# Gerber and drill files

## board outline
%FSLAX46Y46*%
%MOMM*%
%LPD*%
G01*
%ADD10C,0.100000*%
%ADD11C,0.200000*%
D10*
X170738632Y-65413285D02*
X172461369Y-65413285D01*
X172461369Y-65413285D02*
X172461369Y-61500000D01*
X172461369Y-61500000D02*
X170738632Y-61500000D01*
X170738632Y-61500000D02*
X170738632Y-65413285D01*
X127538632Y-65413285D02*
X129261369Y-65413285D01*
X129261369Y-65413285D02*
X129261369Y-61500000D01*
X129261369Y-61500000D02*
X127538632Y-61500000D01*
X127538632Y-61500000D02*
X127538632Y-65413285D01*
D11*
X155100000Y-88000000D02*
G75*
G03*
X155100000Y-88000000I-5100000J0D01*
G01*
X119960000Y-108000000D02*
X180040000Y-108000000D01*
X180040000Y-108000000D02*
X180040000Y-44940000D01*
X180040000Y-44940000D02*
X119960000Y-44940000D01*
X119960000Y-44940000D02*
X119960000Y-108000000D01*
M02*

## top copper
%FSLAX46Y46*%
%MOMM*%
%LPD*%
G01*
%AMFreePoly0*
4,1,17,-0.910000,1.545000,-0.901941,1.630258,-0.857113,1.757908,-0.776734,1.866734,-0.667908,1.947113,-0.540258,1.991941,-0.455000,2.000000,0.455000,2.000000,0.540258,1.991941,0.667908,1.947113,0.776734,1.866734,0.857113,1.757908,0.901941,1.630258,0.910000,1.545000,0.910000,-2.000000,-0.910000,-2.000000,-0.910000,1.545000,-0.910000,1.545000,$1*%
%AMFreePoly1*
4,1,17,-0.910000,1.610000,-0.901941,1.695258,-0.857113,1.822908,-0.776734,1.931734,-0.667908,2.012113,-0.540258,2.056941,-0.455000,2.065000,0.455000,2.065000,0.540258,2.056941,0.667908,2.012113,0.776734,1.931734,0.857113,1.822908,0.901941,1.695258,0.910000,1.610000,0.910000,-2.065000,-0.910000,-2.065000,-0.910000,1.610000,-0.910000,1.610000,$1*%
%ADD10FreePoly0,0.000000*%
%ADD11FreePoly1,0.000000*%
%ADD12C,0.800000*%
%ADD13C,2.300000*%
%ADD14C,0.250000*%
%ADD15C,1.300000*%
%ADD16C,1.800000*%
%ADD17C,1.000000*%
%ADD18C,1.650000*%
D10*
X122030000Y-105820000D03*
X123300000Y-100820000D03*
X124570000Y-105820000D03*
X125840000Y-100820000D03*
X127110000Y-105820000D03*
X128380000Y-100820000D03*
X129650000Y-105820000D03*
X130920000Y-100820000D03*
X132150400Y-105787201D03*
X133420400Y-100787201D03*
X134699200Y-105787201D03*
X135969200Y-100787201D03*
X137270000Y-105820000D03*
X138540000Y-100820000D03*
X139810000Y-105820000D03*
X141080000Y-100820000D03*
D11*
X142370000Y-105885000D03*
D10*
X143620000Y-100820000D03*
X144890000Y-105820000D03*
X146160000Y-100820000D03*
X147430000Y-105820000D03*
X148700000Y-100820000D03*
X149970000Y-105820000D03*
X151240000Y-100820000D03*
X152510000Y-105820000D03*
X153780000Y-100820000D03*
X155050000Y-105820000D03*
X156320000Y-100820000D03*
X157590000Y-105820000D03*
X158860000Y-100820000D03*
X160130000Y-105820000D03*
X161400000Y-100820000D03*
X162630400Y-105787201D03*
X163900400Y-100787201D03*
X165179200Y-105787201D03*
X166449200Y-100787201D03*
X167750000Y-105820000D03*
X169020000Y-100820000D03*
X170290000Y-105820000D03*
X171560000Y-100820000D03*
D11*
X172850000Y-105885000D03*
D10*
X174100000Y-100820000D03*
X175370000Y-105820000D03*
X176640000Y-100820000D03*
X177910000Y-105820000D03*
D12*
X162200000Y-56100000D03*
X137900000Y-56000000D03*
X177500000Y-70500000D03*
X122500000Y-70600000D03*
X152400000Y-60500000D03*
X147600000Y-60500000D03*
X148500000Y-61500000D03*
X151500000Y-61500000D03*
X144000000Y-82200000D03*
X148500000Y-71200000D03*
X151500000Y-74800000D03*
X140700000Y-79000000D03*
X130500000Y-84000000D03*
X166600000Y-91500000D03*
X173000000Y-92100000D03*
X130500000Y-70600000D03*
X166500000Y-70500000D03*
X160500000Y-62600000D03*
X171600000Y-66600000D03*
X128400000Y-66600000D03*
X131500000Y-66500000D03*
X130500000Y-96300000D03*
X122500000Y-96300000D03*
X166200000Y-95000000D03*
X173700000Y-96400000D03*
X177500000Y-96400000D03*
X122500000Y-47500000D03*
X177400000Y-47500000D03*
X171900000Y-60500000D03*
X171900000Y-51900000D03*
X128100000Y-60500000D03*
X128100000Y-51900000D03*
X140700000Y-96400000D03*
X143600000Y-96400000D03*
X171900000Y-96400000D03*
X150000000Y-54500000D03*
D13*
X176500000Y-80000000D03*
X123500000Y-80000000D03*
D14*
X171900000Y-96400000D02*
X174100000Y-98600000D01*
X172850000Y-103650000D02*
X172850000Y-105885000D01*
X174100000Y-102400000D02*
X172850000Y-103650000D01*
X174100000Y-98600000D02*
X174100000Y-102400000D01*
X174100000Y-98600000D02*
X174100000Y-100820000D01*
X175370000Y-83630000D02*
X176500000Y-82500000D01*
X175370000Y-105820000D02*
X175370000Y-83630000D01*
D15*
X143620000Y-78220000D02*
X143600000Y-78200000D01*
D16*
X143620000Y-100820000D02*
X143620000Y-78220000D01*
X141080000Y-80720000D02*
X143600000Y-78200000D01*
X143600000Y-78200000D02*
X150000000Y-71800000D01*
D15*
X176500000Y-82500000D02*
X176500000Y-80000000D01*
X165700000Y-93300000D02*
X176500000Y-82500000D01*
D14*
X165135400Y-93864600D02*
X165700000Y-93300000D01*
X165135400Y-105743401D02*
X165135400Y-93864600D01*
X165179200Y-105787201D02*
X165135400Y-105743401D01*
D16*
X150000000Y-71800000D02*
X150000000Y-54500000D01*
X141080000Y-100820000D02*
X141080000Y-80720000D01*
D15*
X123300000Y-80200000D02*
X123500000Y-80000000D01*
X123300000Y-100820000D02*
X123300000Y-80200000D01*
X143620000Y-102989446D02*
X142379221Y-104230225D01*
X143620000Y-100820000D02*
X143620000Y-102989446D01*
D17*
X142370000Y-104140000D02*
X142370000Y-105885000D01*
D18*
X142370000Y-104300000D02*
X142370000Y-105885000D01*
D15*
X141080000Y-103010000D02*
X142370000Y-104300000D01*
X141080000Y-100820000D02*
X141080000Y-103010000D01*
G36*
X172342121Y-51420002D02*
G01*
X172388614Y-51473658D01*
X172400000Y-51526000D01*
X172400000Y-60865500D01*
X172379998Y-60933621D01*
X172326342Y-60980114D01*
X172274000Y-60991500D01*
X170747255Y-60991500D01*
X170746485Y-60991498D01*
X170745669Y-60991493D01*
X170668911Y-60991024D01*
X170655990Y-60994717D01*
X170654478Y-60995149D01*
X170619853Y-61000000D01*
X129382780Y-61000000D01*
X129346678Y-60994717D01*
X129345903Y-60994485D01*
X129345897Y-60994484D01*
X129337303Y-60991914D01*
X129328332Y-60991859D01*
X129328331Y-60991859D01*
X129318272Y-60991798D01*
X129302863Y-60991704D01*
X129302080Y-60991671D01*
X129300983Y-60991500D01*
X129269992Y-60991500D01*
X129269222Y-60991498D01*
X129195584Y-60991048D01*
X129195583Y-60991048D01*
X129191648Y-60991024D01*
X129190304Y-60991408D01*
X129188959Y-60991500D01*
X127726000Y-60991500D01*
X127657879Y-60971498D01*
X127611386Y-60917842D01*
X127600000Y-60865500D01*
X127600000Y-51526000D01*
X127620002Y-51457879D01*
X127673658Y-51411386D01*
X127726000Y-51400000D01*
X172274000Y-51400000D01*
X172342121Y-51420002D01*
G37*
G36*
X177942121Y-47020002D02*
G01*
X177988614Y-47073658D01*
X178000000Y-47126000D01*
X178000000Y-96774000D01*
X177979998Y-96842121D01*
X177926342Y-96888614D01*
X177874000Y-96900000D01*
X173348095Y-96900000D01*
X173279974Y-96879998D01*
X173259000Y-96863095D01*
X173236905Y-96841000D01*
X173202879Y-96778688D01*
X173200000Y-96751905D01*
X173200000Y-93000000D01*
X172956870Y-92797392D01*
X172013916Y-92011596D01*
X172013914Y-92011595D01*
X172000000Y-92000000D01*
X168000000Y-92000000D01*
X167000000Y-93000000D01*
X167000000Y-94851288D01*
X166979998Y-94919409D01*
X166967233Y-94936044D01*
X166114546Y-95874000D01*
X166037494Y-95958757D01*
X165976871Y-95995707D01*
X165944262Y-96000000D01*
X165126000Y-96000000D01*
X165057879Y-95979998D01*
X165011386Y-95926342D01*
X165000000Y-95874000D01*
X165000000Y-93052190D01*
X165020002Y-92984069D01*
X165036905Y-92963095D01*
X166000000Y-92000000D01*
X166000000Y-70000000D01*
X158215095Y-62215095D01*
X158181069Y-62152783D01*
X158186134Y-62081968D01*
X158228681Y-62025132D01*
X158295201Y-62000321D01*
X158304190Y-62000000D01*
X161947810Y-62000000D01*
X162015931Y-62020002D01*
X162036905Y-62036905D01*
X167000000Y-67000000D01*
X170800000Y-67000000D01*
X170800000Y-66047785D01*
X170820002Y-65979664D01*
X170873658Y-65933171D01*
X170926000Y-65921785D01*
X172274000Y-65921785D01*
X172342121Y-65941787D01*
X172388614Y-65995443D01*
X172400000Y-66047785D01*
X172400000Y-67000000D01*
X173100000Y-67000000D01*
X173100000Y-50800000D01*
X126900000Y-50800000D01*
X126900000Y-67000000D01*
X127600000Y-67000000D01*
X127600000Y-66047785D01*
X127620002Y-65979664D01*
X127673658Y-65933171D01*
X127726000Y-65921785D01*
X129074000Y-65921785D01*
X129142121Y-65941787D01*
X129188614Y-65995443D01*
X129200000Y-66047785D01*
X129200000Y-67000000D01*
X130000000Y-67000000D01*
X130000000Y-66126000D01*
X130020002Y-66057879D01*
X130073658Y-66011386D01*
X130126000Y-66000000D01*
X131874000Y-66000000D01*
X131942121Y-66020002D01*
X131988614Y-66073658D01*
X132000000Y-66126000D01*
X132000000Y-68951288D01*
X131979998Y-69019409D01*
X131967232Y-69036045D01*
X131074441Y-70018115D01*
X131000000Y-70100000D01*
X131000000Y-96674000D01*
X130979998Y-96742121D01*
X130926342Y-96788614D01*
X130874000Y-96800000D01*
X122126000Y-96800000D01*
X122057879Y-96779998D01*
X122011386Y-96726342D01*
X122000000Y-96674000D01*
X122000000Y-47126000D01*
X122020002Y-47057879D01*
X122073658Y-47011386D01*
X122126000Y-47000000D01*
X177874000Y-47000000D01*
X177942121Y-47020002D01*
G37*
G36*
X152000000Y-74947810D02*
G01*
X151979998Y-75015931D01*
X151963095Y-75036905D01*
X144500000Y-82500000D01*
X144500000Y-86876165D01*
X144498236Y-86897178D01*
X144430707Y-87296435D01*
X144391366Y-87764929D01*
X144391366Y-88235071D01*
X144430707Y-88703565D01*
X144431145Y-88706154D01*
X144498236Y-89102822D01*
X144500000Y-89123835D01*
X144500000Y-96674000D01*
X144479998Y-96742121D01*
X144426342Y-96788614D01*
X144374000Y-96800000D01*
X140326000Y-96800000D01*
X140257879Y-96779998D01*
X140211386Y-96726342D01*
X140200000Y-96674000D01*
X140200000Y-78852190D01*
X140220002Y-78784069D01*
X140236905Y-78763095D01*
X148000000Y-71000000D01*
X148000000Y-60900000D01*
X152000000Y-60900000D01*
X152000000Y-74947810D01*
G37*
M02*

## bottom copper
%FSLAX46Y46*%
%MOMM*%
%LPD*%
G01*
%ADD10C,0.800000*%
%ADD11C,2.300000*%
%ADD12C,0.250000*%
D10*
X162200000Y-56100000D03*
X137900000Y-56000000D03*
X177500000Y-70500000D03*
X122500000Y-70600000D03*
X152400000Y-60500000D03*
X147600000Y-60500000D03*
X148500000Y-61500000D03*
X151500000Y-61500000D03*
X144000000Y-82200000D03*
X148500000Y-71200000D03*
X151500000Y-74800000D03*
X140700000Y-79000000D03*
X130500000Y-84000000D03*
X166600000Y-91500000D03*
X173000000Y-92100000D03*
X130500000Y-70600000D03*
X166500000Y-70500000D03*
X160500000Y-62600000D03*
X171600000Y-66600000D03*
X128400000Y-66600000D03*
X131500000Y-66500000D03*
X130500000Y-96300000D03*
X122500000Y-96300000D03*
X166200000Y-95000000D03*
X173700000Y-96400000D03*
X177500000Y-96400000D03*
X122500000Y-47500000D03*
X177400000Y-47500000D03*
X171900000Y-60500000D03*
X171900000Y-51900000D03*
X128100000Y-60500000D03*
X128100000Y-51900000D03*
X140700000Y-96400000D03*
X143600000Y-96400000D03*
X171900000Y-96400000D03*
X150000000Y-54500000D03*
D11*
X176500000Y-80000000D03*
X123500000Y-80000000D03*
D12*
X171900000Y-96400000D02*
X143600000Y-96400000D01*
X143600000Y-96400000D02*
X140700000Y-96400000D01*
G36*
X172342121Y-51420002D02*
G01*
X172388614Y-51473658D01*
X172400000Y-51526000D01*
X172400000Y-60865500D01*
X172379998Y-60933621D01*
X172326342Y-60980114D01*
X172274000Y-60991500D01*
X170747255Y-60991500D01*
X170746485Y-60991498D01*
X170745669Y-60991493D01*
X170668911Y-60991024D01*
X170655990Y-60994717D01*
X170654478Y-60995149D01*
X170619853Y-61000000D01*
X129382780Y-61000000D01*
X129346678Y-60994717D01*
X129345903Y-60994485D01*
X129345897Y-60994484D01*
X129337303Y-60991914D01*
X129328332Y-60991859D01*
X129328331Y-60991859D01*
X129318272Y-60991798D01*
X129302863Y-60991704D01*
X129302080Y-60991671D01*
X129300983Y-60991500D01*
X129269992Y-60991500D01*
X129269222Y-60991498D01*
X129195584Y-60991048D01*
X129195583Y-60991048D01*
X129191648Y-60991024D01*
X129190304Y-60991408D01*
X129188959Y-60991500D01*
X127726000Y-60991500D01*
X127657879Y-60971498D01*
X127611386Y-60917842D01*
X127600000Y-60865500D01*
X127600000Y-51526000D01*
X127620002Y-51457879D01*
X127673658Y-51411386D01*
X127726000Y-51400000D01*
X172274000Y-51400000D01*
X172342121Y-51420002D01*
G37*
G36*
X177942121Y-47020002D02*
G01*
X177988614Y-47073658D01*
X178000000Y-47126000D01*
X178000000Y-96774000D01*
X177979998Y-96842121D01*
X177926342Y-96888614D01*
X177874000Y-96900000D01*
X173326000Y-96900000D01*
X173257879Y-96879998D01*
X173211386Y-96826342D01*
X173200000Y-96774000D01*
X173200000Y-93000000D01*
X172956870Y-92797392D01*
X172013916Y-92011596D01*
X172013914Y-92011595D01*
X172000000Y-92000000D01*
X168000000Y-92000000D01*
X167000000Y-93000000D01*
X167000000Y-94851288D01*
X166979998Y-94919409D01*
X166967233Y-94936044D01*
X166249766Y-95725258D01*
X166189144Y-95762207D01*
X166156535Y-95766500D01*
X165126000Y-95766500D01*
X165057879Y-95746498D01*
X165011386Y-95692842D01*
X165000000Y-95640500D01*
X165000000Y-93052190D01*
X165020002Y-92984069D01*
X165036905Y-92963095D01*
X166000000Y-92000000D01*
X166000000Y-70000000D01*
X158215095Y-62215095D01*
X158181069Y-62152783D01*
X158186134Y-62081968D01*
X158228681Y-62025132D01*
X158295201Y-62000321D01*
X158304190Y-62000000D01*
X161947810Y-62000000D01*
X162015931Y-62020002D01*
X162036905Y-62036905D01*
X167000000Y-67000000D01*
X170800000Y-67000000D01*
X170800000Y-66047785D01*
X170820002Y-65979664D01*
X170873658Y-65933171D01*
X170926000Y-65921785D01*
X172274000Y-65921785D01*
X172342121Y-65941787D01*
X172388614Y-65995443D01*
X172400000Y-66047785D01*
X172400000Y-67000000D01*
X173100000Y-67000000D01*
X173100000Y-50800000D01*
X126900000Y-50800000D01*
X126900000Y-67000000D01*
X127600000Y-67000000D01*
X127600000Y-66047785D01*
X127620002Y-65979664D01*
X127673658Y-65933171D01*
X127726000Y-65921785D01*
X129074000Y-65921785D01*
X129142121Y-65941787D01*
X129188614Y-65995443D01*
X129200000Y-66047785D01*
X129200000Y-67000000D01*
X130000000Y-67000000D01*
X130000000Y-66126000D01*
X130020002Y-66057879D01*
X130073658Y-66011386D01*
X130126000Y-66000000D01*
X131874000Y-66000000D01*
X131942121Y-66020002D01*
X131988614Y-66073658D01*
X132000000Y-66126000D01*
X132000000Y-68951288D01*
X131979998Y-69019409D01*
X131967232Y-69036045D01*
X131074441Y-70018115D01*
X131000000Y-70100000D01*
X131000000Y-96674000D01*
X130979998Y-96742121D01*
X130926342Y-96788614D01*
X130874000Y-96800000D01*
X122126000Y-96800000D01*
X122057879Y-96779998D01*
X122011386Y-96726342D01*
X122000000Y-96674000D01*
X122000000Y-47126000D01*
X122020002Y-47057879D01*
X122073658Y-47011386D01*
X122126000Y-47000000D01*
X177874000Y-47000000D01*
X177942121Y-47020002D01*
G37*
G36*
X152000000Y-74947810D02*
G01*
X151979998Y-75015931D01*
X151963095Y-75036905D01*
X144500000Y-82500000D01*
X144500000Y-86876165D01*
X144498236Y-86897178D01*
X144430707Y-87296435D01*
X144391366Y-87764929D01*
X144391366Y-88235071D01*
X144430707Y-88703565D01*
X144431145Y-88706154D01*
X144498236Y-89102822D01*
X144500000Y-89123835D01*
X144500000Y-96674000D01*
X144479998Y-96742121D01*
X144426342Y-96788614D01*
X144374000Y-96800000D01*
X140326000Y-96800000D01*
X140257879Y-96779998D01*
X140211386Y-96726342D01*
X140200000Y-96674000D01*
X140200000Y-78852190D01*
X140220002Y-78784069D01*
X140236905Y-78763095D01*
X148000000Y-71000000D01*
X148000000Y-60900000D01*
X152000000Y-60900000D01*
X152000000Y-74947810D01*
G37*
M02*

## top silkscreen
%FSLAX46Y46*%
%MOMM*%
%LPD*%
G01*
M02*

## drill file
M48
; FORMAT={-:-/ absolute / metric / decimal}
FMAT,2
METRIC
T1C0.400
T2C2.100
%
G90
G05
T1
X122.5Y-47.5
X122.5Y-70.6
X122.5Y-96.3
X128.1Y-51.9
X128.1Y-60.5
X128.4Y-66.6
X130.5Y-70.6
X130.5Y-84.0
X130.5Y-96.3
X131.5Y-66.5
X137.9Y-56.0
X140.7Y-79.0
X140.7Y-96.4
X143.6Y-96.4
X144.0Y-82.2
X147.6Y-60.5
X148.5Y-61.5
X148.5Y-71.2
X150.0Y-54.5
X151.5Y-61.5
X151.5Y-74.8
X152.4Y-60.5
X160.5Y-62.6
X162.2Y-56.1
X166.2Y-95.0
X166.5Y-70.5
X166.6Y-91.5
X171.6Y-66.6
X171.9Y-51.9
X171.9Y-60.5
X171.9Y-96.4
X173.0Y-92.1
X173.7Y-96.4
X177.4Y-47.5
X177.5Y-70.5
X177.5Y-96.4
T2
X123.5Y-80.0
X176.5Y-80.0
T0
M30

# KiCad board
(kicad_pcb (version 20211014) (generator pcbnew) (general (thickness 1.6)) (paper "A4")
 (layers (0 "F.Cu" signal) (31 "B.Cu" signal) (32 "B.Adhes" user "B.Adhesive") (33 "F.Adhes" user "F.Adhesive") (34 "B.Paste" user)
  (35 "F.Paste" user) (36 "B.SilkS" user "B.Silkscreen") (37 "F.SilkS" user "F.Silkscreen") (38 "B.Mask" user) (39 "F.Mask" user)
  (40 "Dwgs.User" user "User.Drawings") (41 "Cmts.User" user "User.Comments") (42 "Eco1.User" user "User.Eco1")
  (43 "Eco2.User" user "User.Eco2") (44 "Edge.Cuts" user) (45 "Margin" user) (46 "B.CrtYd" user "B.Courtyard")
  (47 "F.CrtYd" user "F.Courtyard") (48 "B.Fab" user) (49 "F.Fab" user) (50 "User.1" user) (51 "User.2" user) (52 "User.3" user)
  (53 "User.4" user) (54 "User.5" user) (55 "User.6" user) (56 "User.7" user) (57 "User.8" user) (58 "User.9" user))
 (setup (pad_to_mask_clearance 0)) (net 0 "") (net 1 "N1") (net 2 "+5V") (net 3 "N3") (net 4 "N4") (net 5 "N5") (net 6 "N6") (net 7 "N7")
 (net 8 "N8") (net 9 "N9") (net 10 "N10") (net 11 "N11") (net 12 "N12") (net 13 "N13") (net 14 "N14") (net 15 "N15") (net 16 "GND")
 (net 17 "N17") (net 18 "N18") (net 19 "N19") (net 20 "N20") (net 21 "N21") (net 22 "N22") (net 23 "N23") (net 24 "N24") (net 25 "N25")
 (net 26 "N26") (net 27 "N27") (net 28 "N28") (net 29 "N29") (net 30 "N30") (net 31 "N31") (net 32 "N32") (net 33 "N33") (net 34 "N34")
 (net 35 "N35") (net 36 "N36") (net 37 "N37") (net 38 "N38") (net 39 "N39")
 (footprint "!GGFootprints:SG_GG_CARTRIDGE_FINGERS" (layer "F.Cu") (at 150 103.34) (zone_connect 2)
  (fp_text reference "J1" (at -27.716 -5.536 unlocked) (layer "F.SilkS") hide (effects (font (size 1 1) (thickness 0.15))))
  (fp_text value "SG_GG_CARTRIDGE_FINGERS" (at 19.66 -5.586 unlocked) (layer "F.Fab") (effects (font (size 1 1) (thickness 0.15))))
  (pad "1" connect roundrect (at -27.97 2.48) (size 1.82 4) (layers "F.Cu" "F.Mask") (roundrect_rratio 0.25) (chamfer_ratio 0)
   (chamfer bottom_left bottom_right) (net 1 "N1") (zone_connect 2))
  (pad "2" connect roundrect (at -26.7 -2.52) (size 1.82 4) (layers "F.Cu" "F.Mask") (roundrect_rratio 0.25) (chamfer_ratio 0)
   (chamfer bottom_left bottom_right) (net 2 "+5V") (zone_connect 2))
  (pad "3" connect roundrect (at -25.43 2.48) (size 1.82 4) (layers "F.Cu" "F.Mask") (roundrect_rratio 0.25) (chamfer_ratio 0)
   (chamfer bottom_left bottom_right) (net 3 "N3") (zone_connect 2))
  (pad "4" connect roundrect (at -24.16 -2.52) (size 1.82 4) (layers "F.Cu" "F.Mask") (roundrect_rratio 0.25) (chamfer_ratio 0)
   (chamfer bottom_left bottom_right) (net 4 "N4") (zone_connect 2))
  (pad "5" connect roundrect (at -22.89 2.48) (size 1.82 4) (layers "F.Cu" "F.Mask") (roundrect_rratio 0.25) (chamfer_ratio 0)
   (chamfer bottom_left bottom_right) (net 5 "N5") (zone_connect 2))
  (pad "6" connect roundrect (at -21.62 -2.52) (size 1.82 4) (layers "F.Cu" "F.Mask") (roundrect_rratio 0.25) (chamfer_ratio 0)
   (chamfer bottom_left bottom_right) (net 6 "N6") (zone_connect 2))
  (pad "7" connect roundrect (at -20.35 2.48) (size 1.82 4) (layers "F.Cu" "F.Mask") (roundrect_rratio 0.25) (chamfer_ratio 0)
   (chamfer bottom_left bottom_right) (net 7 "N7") (zone_connect 2))
  (pad "8" connect roundrect (at -19.08 -2.52) (size 1.82 4) (layers "F.Cu" "F.Mask") (roundrect_rratio 0.25) (chamfer_ratio 0)
   (chamfer bottom_left bottom_right) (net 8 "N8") (zone_connect 2))
  (pad "9" connect roundrect (at -17.8496 2.447201) (size 1.82 4) (layers "F.Cu" "F.Mask") (roundrect_rratio 0.25) (chamfer_ratio 0)
   (chamfer bottom_left bottom_right) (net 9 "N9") (zone_connect 2))
  (pad "10" connect roundrect (at -16.5796 -2.552799) (size 1.82 4) (layers "F.Cu" "F.Mask") (roundrect_rratio 0.25) (chamfer_ratio 0)
   (chamfer bottom_left bottom_right) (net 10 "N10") (zone_connect 2))
  (pad "11" connect roundrect (at -15.3008 2.447201) (size 1.82 4) (layers "F.Cu" "F.Mask") (roundrect_rratio 0.25) (chamfer_ratio 0)
   (chamfer bottom_left bottom_right) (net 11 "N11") (zone_connect 2))
  (pad "12" connect roundrect (at -14.0308 -2.552799) (size 1.82 4) (layers "F.Cu" "F.Mask") (roundrect_rratio 0.25) (chamfer_ratio 0)
   (chamfer bottom_left bottom_right) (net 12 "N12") (zone_connect 2))
  (pad "13" connect roundrect (at -12.73 2.48) (size 1.82 4) (layers "F.Cu" "F.Mask") (roundrect_rratio 0.25) (chamfer_ratio 0)
   (chamfer bottom_left bottom_right) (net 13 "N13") (zone_connect 2))
  (pad "14" connect roundrect (at -11.46 -2.52) (size 1.82 4) (layers "F.Cu" "F.Mask") (roundrect_rratio 0.25) (chamfer_ratio 0)
   (chamfer bottom_left bottom_right) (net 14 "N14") (zone_connect 2))
  (pad "15" connect roundrect (at -10.19 2.48) (size 1.82 4) (layers "F.Cu" "F.Mask") (roundrect_rratio 0.25) (chamfer_ratio 0)
   (chamfer bottom_left bottom_right) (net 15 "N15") (zone_connect 2))
  (pad "16" connect roundrect (at -8.92 -2.52) (size 1.82 4) (layers "F.Cu" "F.Mask") (roundrect_rratio 0.25) (chamfer_ratio 0)
   (chamfer bottom_left bottom_right) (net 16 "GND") (zone_connect 2))
  (pad "17" connect roundrect (at -7.63 2.545) (size 1.82 4.13) (layers "F.Cu" "F.Mask") (roundrect_rratio 0.25) (chamfer_ratio 0)
   (chamfer bottom_left bottom_right) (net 16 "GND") (zone_connect 2))
  (pad "18" connect roundrect (at -6.38 -2.52) (size 1.82 4) (layers "F.Cu" "F.Mask") (roundrect_rratio 0.25) (chamfer_ratio 0)
   (chamfer bottom_left bottom_right) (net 16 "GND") (zone_connect 2))
  (pad "19" connect roundrect (at -5.11 2.48) (size 1.82 4) (layers "F.Cu" "F.Mask") (roundrect_rratio 0.25) (chamfer_ratio 0)
   (chamfer bottom_left bottom_right) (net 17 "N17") (zone_connect 2))
  (pad "20" connect roundrect (at -3.84 -2.52) (size 1.82 4) (layers "F.Cu" "F.Mask") (roundrect_rratio 0.25) (chamfer_ratio 0)
   (chamfer bottom_left bottom_right) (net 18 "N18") (zone_connect 2))
  (pad "21" connect roundrect (at -2.57 2.48) (size 1.82 4) (layers "F.Cu" "F.Mask") (roundrect_rratio 0.25) (chamfer_ratio 0)
   (chamfer bottom_left bottom_right) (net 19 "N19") (zone_connect 2))
  (pad "22" connect roundrect (at -1.3 -2.52) (size 1.82 4) (layers "F.Cu" "F.Mask") (roundrect_rratio 0.25) (chamfer_ratio 0)
   (chamfer bottom_left bottom_right) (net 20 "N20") (zone_connect 2))
  (pad "23" connect roundrect (at -0.03 2.48) (size 1.82 4) (layers "F.Cu" "F.Mask") (roundrect_rratio 0.25) (chamfer_ratio 0)
   (chamfer bottom_left bottom_right) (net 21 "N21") (zone_connect 2))
  (pad "24" connect roundrect (at 1.24 -2.52) (size 1.82 4) (layers "F.Cu" "F.Mask") (roundrect_rratio 0.25) (chamfer_ratio 0)
   (chamfer bottom_left bottom_right) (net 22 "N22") (zone_connect 2))
  (pad "25" connect roundrect (at 2.51 2.48) (size 1.82 4) (layers "F.Cu" "F.Mask") (roundrect_rratio 0.25) (chamfer_ratio 0)
   (chamfer bottom_left bottom_right) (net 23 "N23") (zone_connect 2))
  (pad "26" connect roundrect (at 3.78 -2.52) (size 1.82 4) (layers "F.Cu" "F.Mask") (roundrect_rratio 0.25) (chamfer_ratio 0)
   (chamfer bottom_left bottom_right) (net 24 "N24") (zone_connect 2))
  (pad "27" connect roundrect (at 5.05 2.48) (size 1.82 4) (layers "F.Cu" "F.Mask") (roundrect_rratio 0.25) (chamfer_ratio 0)
   (chamfer bottom_left bottom_right) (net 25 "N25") (zone_connect 2))
  (pad "28" connect roundrect (at 6.32 -2.52) (size 1.82 4) (layers "F.Cu" "F.Mask") (roundrect_rratio 0.25) (chamfer_ratio 0)
   (chamfer bottom_left bottom_right) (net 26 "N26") (zone_connect 2))
  (pad "29" connect roundrect (at 7.59 2.48) (size 1.82 4) (layers "F.Cu" "F.Mask") (roundrect_rratio 0.25) (chamfer_ratio 0)
   (chamfer bottom_left bottom_right) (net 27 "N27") (zone_connect 2))
  (pad "30" connect roundrect (at 8.86 -2.52) (size 1.82 4) (layers "F.Cu" "F.Mask") (roundrect_rratio 0.25) (chamfer_ratio 0)
   (chamfer bottom_left bottom_right) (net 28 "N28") (zone_connect 2))
  (pad "31" connect roundrect (at 10.13 2.48) (size 1.82 4) (layers "F.Cu" "F.Mask") (roundrect_rratio 0.25) (chamfer_ratio 0)
   (chamfer bottom_left bottom_right) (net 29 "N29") (zone_connect 2))
  (pad "32" connect roundrect (at 11.4 -2.52) (size 1.82 4) (layers "F.Cu" "F.Mask") (roundrect_rratio 0.25) (chamfer_ratio 0)
   (chamfer bottom_left bottom_right) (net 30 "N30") (zone_connect 2))
  (pad "33" connect roundrect (at 12.6304 2.447201) (size 1.82 4) (layers "F.Cu" "F.Mask") (roundrect_rratio 0.25) (chamfer_ratio 0)
   (chamfer bottom_left bottom_right) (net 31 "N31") (zone_connect 2))
  (pad "34" connect roundrect (at 13.9004 -2.552799) (size 1.82 4) (layers "F.Cu" "F.Mask") (roundrect_rratio 0.25) (chamfer_ratio 0)
   (chamfer bottom_left bottom_right) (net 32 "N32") (zone_connect 2))
  (pad "35" connect roundrect (at 15.1792 2.447201) (size 1.82 4) (layers "F.Cu" "F.Mask") (roundrect_rratio 0.25) (chamfer_ratio 0)
   (chamfer bottom_left bottom_right) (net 2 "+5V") (zone_connect 2))
  (pad "36" connect roundrect (at 16.4492 -2.552799) (size 1.82 4) (layers "F.Cu" "F.Mask") (roundrect_rratio 0.25) (chamfer_ratio 0)
   (chamfer bottom_left bottom_right) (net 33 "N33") (zone_connect 2))
  (pad "37" connect roundrect (at 17.75 2.48) (size 1.82 4) (layers "F.Cu" "F.Mask") (roundrect_rratio 0.25) (chamfer_ratio 0)
   (chamfer bottom_left bottom_right) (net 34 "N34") (zone_connect 2))
  (pad "38" connect roundrect (at 19.02 -2.52) (size 1.82 4) (layers "F.Cu" "F.Mask") (roundrect_rratio 0.25) (chamfer_ratio 0)
   (chamfer bottom_left bottom_right) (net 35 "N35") (zone_connect 2))
  (pad "39" connect roundrect (at 20.29 2.48) (size 1.82 4) (layers "F.Cu" "F.Mask") (roundrect_rratio 0.25) (chamfer_ratio 0)
   (chamfer bottom_left bottom_right) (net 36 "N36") (zone_connect 2))
  (pad "40" connect roundrect (at 21.56 -2.52) (size 1.82 4) (layers "F.Cu" "F.Mask") (roundrect_rratio 0.25) (chamfer_ratio 0)
   (chamfer bottom_left bottom_right) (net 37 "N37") (zone_connect 2))
  (pad "41" connect roundrect (at 22.85 2.545) (size 1.82 4.13) (layers "F.Cu" "F.Mask") (roundrect_rratio 0.25) (chamfer_ratio 0)
   (chamfer bottom_left bottom_right) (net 16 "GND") (zone_connect 2))
  (pad "42" connect roundrect (at 24.1 -2.52) (size 1.82 4) (layers "F.Cu" "F.Mask") (roundrect_rratio 0.25) (chamfer_ratio 0)
   (chamfer bottom_left bottom_right) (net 16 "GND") (zone_connect 2))
  (pad "43" connect roundrect (at 25.37 2.48) (size 1.82 4) (layers "F.Cu" "F.Mask") (roundrect_rratio 0.25) (chamfer_ratio 0)
   (chamfer bottom_left bottom_right) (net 2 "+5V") (zone_connect 2))
  (pad "44" connect roundrect (at 26.64 -2.52) (size 1.82 4) (layers "F.Cu" "F.Mask") (roundrect_rratio 0.25) (chamfer_ratio 0)
   (chamfer bottom_left bottom_right) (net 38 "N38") (zone_connect 2))
  (pad "45" connect roundrect (at 27.91 2.48) (size 1.82 4) (layers "F.Cu" "F.Mask") (roundrect_rratio 0.25) (chamfer_ratio 0)
   (chamfer bottom_left bottom_right) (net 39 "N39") (zone_connect 2)))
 (gr_rect (start 119.96 108) (end 180.04 44.94) (layer "Edge.Cuts") (width 0.2) (fill none))
 (gr_circle (center 150 88) (end 155.1 88) (layer "Edge.Cuts") (width 0.2) (fill none))
 (gr_rect (start 170.738632 65.413285) (end 172.461369 61.5) (layer "Edge.Cuts") (width 0.1) (fill none))
 (gr_rect (start 127.538632 65.413285) (end 129.261369 61.5) (layer "Edge.Cuts") (width 0.1) (fill none))
 (segment (start 123.3 80.2) (end 123.5 80) (width 1.3) (layer "F.Cu") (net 2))
 (segment (start 123.3 100.82) (end 123.3 80.2) (width 1.3) (layer "F.Cu") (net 2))
 (segment (start 165.1354 93.8646) (end 165.7 93.3) (width 0.25) (layer "F.Cu") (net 2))
 (segment (start 175.37 105.82) (end 175.37 83.63) (width 0.25) (layer "F.Cu") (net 2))
 (segment (start 165.1792 105.787201) (end 165.1354 105.743401) (width 0.25) (layer "F.Cu") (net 2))
 (segment (start 176.5 82.5) (end 176.5 80) (width 1.3) (layer "F.Cu") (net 2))
 (segment (start 165.1354 105.743401) (end 165.1354 93.8646) (width 0.25) (layer "F.Cu") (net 2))
 (segment (start 175.37 83.63) (end 176.5 82.5) (width 0.25) (layer "F.Cu") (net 2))
 (segment (start 165.7 93.3) (end 176.5 82.5) (width 1.3) (layer "F.Cu") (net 2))
 (via (at 130.5 84) (size 0.8) (drill 0.4) (layers "F.Cu" "B.Cu") (free) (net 2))
 (via (at 122.5 47.5) (size 0.8) (drill 0.4) (layers "F.Cu" "B.Cu") (free) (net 2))
 (via (at 122.5 96.3) (size 0.8) (drill 0.4) (layers "F.Cu" "B.Cu") (free) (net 2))
 (via (at 173.7 96.4) (size 0.8) (drill 0.4) (layers "F.Cu" "B.Cu") (free) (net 2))
 (via (at 173 92.1) (size 0.8) (drill 0.4) (layers "F.Cu" "B.Cu") (free) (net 2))
 (via (at 166.5 70.5) (size 0.8) (drill 0.4) (layers "F.Cu" "B.Cu") (free) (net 2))
 (via (at 160.5 62.6) (size 0.8) (drill 0.4) (layers "F.Cu" "B.Cu") (free) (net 2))
 (via (at 166.6 91.5) (size 0.8) (drill 0.4) (layers "F.Cu" "B.Cu") (free) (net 2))
 (via (at 177.5 96.4) (size 0.8) (drill 0.4) (layers "F.Cu" "B.Cu") (free) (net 2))
 (via (at 176.5 80) (size 2.3) (drill 2.1) (layers "F.Cu" "B.Cu") (free) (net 2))
 (via (at 122.5 70.6) (size 0.8) (drill 0.4) (layers "F.Cu" "B.Cu") (free) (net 2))
 (via (at 130.5 70.6) (size 0.8) (drill 0.4) (layers "F.Cu" "B.Cu") (free) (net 2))
 (via (at 128.4 66.6) (size 0.8) (drill 0.4) (layers "F.Cu" "B.Cu") (free) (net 2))
 (via (at 130.5 96.3) (size 0.8) (drill 0.4) (layers "F.Cu" "B.Cu") (free) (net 2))
 (via (at 166.2 95) (size 0.8) (drill 0.4) (layers "F.Cu" "B.Cu") (free) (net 2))
 (via (at 171.6 66.6) (size 0.8) (drill 0.4) (layers "F.Cu" "B.Cu") (free) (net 2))
 (via (at 131.5 66.5) (size 0.8) (drill 0.4) (layers "F.Cu" "B.Cu") (free) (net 2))
 (via (at 123.5 80) (size 2.3) (drill 2.1) (layers "F.Cu" "B.Cu") (free) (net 2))
 (via (at 177.5 70.5) (size 0.8) (drill 0.4) (layers "F.Cu" "B.Cu") (free) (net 2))
 (via (at 177.4 47.5) (size 0.8) (drill 0.4) (layers "F.Cu" "B.Cu") (free) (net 2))
 (segment (start 141.08 100.82) (end 141.08 103.01) (width 1.3) (layer "F.Cu") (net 16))
 (segment (start 143.62 100.82) (end 143.62 78.22) (width 1.8) (layer "F.Cu") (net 16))
 (segment (start 143.62 100.82) (end 143.62 102.989446) (width 1.3) (layer "F.Cu") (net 16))
 (segment (start 172.85 103.65) (end 172.85 105.885) (width 0.25) (layer "F.Cu") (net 16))
 (segment (start 142.37 104.3) (end 142.37 105.885) (width 1.65) (layer "F.Cu") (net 16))
 (segment (start 171.9 96.4) (end 174.1 98.6) (width 0.25) (layer "F.Cu") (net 16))
 (segment (start 143.6 78.2) (end 150 71.8) (width 1.8) (layer "F.Cu") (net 16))
 (segment (start 150 71.8) (end 150 54.5) (width 1.8) (layer "F.Cu") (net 16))
 (segment (start 141.08 103.01) (end 142.37 104.3) (width 1.3) (layer "F.Cu") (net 16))
 (segment (start 143.62 78.22) (end 143.6 78.2) (width 1.3) (layer "F.Cu") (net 16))
 (segment (start 141.08 100.82) (end 141.08 80.72) (width 1.8) (layer "F.Cu") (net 16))
 (segment (start 174.1 98.6) (end 174.1 102.4) (width 0.25) (layer "F.Cu") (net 16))
 (segment (start 142.37 104.14) (end 142.37 105.885) (width 1) (layer "F.Cu") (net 16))
 (segment (start 141.08 80.72) (end 143.6 78.2) (width 1.8) (layer "F.Cu") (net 16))
 (segment (start 174.1 102.4) (end 172.85 103.65) (width 0.25) (layer "F.Cu") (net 16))
 (segment (start 174.1 98.6) (end 174.1 100.82) (width 0.25) (layer "F.Cu") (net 16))
 (segment (start 143.62 102.989446) (end 142.379221 104.230225) (width 1.3) (layer "F.Cu") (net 16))
 (via (at 148.5 71.2) (size 0.8) (drill 0.4) (layers "F.Cu" "B.Cu") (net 16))
 (via (at 171.9 51.9) (size 0.8) (drill 0.4) (layers "F.Cu" "B.Cu") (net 16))
 (via (at 143.6 96.4) (size 0.8) (drill 0.4) (layers "F.Cu" "B.Cu") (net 16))
 (via (at 171.9 60.5) (size 0.8) (drill 0.4) (layers "F.Cu" "B.Cu") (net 16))
 (via (at 150 54.5) (size 0.8) (drill 0.4) (layers "F.Cu" "B.Cu") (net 16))
 (via (at 152.4 60.5) (size 0.8) (drill 0.4) (layers "F.Cu" "B.Cu") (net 16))
 (via (at 162.2 56.1) (size 0.8) (drill 0.4) (layers "F.Cu" "B.Cu") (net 16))
 (via (at 137.9 56) (size 0.8) (drill 0.4) (layers "F.Cu" "B.Cu") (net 16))
 (via (at 147.6 60.5) (size 0.8) (drill 0.4) (layers "F.Cu" "B.Cu") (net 16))
 (via (at 140.7 96.4) (size 0.8) (drill 0.4) (layers "F.Cu" "B.Cu") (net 16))
 (via (at 148.5 61.5) (size 0.8) (drill 0.4) (layers "F.Cu" "B.Cu") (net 16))
 (via (at 171.9 96.4) (size 0.8) (drill 0.4) (layers "F.Cu" "B.Cu") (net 16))
 (via (at 140.7 79) (size 0.8) (drill 0.4) (layers "F.Cu" "B.Cu") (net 16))
 (via (at 151.5 74.8) (size 0.8) (drill 0.4) (layers "F.Cu" "B.Cu") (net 16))
 (via (at 128.1 51.9) (size 0.8) (drill 0.4) (layers "F.Cu" "B.Cu") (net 16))
 (via (at 151.5 61.5) (size 0.8) (drill 0.4) (layers "F.Cu" "B.Cu") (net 16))
 (via (at 144 82.2) (size 0.8) (drill 0.4) (layers "F.Cu" "B.Cu") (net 16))
 (via (at 128.1 60.5) (size 0.8) (drill 0.4) (layers "F.Cu" "B.Cu") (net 16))
 (segment (start 143.6 96.4) (end 140.7 96.4) (width 0.25) (layer "B.Cu") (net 16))
 (segment (start 171.9 96.4) (end 143.6 96.4) (width 0.25) (layer "B.Cu") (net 16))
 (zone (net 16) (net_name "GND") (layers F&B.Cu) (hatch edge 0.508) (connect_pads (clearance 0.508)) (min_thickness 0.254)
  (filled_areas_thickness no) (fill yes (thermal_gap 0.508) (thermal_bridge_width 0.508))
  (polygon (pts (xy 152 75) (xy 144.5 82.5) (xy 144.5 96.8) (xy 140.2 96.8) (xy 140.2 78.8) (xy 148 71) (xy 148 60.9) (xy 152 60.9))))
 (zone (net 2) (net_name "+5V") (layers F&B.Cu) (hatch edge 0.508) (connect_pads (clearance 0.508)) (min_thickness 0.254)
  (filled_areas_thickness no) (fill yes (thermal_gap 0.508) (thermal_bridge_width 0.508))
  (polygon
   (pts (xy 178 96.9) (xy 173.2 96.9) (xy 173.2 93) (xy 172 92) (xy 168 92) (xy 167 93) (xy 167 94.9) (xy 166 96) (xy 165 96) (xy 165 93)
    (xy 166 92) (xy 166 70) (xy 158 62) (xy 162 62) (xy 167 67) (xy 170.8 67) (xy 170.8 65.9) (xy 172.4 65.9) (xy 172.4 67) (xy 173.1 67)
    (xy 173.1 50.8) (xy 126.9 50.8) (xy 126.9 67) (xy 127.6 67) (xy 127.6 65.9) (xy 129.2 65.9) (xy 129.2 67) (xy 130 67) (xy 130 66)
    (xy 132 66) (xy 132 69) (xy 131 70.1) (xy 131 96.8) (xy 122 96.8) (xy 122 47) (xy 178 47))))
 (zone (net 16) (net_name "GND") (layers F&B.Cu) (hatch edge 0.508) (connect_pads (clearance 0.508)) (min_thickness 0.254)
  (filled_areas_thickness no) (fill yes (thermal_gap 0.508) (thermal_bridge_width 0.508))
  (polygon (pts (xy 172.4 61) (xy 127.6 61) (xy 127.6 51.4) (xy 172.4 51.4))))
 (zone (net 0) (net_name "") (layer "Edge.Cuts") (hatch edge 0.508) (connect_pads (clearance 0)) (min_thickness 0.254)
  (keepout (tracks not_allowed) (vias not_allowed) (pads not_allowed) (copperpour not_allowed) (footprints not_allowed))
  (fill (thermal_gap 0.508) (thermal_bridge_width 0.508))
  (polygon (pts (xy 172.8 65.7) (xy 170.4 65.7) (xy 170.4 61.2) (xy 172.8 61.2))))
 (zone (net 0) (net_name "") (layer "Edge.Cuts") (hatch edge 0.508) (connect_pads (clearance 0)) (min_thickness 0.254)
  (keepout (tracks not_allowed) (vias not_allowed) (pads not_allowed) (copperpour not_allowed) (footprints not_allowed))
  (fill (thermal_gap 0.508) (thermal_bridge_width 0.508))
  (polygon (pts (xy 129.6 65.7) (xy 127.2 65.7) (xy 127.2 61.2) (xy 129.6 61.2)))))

